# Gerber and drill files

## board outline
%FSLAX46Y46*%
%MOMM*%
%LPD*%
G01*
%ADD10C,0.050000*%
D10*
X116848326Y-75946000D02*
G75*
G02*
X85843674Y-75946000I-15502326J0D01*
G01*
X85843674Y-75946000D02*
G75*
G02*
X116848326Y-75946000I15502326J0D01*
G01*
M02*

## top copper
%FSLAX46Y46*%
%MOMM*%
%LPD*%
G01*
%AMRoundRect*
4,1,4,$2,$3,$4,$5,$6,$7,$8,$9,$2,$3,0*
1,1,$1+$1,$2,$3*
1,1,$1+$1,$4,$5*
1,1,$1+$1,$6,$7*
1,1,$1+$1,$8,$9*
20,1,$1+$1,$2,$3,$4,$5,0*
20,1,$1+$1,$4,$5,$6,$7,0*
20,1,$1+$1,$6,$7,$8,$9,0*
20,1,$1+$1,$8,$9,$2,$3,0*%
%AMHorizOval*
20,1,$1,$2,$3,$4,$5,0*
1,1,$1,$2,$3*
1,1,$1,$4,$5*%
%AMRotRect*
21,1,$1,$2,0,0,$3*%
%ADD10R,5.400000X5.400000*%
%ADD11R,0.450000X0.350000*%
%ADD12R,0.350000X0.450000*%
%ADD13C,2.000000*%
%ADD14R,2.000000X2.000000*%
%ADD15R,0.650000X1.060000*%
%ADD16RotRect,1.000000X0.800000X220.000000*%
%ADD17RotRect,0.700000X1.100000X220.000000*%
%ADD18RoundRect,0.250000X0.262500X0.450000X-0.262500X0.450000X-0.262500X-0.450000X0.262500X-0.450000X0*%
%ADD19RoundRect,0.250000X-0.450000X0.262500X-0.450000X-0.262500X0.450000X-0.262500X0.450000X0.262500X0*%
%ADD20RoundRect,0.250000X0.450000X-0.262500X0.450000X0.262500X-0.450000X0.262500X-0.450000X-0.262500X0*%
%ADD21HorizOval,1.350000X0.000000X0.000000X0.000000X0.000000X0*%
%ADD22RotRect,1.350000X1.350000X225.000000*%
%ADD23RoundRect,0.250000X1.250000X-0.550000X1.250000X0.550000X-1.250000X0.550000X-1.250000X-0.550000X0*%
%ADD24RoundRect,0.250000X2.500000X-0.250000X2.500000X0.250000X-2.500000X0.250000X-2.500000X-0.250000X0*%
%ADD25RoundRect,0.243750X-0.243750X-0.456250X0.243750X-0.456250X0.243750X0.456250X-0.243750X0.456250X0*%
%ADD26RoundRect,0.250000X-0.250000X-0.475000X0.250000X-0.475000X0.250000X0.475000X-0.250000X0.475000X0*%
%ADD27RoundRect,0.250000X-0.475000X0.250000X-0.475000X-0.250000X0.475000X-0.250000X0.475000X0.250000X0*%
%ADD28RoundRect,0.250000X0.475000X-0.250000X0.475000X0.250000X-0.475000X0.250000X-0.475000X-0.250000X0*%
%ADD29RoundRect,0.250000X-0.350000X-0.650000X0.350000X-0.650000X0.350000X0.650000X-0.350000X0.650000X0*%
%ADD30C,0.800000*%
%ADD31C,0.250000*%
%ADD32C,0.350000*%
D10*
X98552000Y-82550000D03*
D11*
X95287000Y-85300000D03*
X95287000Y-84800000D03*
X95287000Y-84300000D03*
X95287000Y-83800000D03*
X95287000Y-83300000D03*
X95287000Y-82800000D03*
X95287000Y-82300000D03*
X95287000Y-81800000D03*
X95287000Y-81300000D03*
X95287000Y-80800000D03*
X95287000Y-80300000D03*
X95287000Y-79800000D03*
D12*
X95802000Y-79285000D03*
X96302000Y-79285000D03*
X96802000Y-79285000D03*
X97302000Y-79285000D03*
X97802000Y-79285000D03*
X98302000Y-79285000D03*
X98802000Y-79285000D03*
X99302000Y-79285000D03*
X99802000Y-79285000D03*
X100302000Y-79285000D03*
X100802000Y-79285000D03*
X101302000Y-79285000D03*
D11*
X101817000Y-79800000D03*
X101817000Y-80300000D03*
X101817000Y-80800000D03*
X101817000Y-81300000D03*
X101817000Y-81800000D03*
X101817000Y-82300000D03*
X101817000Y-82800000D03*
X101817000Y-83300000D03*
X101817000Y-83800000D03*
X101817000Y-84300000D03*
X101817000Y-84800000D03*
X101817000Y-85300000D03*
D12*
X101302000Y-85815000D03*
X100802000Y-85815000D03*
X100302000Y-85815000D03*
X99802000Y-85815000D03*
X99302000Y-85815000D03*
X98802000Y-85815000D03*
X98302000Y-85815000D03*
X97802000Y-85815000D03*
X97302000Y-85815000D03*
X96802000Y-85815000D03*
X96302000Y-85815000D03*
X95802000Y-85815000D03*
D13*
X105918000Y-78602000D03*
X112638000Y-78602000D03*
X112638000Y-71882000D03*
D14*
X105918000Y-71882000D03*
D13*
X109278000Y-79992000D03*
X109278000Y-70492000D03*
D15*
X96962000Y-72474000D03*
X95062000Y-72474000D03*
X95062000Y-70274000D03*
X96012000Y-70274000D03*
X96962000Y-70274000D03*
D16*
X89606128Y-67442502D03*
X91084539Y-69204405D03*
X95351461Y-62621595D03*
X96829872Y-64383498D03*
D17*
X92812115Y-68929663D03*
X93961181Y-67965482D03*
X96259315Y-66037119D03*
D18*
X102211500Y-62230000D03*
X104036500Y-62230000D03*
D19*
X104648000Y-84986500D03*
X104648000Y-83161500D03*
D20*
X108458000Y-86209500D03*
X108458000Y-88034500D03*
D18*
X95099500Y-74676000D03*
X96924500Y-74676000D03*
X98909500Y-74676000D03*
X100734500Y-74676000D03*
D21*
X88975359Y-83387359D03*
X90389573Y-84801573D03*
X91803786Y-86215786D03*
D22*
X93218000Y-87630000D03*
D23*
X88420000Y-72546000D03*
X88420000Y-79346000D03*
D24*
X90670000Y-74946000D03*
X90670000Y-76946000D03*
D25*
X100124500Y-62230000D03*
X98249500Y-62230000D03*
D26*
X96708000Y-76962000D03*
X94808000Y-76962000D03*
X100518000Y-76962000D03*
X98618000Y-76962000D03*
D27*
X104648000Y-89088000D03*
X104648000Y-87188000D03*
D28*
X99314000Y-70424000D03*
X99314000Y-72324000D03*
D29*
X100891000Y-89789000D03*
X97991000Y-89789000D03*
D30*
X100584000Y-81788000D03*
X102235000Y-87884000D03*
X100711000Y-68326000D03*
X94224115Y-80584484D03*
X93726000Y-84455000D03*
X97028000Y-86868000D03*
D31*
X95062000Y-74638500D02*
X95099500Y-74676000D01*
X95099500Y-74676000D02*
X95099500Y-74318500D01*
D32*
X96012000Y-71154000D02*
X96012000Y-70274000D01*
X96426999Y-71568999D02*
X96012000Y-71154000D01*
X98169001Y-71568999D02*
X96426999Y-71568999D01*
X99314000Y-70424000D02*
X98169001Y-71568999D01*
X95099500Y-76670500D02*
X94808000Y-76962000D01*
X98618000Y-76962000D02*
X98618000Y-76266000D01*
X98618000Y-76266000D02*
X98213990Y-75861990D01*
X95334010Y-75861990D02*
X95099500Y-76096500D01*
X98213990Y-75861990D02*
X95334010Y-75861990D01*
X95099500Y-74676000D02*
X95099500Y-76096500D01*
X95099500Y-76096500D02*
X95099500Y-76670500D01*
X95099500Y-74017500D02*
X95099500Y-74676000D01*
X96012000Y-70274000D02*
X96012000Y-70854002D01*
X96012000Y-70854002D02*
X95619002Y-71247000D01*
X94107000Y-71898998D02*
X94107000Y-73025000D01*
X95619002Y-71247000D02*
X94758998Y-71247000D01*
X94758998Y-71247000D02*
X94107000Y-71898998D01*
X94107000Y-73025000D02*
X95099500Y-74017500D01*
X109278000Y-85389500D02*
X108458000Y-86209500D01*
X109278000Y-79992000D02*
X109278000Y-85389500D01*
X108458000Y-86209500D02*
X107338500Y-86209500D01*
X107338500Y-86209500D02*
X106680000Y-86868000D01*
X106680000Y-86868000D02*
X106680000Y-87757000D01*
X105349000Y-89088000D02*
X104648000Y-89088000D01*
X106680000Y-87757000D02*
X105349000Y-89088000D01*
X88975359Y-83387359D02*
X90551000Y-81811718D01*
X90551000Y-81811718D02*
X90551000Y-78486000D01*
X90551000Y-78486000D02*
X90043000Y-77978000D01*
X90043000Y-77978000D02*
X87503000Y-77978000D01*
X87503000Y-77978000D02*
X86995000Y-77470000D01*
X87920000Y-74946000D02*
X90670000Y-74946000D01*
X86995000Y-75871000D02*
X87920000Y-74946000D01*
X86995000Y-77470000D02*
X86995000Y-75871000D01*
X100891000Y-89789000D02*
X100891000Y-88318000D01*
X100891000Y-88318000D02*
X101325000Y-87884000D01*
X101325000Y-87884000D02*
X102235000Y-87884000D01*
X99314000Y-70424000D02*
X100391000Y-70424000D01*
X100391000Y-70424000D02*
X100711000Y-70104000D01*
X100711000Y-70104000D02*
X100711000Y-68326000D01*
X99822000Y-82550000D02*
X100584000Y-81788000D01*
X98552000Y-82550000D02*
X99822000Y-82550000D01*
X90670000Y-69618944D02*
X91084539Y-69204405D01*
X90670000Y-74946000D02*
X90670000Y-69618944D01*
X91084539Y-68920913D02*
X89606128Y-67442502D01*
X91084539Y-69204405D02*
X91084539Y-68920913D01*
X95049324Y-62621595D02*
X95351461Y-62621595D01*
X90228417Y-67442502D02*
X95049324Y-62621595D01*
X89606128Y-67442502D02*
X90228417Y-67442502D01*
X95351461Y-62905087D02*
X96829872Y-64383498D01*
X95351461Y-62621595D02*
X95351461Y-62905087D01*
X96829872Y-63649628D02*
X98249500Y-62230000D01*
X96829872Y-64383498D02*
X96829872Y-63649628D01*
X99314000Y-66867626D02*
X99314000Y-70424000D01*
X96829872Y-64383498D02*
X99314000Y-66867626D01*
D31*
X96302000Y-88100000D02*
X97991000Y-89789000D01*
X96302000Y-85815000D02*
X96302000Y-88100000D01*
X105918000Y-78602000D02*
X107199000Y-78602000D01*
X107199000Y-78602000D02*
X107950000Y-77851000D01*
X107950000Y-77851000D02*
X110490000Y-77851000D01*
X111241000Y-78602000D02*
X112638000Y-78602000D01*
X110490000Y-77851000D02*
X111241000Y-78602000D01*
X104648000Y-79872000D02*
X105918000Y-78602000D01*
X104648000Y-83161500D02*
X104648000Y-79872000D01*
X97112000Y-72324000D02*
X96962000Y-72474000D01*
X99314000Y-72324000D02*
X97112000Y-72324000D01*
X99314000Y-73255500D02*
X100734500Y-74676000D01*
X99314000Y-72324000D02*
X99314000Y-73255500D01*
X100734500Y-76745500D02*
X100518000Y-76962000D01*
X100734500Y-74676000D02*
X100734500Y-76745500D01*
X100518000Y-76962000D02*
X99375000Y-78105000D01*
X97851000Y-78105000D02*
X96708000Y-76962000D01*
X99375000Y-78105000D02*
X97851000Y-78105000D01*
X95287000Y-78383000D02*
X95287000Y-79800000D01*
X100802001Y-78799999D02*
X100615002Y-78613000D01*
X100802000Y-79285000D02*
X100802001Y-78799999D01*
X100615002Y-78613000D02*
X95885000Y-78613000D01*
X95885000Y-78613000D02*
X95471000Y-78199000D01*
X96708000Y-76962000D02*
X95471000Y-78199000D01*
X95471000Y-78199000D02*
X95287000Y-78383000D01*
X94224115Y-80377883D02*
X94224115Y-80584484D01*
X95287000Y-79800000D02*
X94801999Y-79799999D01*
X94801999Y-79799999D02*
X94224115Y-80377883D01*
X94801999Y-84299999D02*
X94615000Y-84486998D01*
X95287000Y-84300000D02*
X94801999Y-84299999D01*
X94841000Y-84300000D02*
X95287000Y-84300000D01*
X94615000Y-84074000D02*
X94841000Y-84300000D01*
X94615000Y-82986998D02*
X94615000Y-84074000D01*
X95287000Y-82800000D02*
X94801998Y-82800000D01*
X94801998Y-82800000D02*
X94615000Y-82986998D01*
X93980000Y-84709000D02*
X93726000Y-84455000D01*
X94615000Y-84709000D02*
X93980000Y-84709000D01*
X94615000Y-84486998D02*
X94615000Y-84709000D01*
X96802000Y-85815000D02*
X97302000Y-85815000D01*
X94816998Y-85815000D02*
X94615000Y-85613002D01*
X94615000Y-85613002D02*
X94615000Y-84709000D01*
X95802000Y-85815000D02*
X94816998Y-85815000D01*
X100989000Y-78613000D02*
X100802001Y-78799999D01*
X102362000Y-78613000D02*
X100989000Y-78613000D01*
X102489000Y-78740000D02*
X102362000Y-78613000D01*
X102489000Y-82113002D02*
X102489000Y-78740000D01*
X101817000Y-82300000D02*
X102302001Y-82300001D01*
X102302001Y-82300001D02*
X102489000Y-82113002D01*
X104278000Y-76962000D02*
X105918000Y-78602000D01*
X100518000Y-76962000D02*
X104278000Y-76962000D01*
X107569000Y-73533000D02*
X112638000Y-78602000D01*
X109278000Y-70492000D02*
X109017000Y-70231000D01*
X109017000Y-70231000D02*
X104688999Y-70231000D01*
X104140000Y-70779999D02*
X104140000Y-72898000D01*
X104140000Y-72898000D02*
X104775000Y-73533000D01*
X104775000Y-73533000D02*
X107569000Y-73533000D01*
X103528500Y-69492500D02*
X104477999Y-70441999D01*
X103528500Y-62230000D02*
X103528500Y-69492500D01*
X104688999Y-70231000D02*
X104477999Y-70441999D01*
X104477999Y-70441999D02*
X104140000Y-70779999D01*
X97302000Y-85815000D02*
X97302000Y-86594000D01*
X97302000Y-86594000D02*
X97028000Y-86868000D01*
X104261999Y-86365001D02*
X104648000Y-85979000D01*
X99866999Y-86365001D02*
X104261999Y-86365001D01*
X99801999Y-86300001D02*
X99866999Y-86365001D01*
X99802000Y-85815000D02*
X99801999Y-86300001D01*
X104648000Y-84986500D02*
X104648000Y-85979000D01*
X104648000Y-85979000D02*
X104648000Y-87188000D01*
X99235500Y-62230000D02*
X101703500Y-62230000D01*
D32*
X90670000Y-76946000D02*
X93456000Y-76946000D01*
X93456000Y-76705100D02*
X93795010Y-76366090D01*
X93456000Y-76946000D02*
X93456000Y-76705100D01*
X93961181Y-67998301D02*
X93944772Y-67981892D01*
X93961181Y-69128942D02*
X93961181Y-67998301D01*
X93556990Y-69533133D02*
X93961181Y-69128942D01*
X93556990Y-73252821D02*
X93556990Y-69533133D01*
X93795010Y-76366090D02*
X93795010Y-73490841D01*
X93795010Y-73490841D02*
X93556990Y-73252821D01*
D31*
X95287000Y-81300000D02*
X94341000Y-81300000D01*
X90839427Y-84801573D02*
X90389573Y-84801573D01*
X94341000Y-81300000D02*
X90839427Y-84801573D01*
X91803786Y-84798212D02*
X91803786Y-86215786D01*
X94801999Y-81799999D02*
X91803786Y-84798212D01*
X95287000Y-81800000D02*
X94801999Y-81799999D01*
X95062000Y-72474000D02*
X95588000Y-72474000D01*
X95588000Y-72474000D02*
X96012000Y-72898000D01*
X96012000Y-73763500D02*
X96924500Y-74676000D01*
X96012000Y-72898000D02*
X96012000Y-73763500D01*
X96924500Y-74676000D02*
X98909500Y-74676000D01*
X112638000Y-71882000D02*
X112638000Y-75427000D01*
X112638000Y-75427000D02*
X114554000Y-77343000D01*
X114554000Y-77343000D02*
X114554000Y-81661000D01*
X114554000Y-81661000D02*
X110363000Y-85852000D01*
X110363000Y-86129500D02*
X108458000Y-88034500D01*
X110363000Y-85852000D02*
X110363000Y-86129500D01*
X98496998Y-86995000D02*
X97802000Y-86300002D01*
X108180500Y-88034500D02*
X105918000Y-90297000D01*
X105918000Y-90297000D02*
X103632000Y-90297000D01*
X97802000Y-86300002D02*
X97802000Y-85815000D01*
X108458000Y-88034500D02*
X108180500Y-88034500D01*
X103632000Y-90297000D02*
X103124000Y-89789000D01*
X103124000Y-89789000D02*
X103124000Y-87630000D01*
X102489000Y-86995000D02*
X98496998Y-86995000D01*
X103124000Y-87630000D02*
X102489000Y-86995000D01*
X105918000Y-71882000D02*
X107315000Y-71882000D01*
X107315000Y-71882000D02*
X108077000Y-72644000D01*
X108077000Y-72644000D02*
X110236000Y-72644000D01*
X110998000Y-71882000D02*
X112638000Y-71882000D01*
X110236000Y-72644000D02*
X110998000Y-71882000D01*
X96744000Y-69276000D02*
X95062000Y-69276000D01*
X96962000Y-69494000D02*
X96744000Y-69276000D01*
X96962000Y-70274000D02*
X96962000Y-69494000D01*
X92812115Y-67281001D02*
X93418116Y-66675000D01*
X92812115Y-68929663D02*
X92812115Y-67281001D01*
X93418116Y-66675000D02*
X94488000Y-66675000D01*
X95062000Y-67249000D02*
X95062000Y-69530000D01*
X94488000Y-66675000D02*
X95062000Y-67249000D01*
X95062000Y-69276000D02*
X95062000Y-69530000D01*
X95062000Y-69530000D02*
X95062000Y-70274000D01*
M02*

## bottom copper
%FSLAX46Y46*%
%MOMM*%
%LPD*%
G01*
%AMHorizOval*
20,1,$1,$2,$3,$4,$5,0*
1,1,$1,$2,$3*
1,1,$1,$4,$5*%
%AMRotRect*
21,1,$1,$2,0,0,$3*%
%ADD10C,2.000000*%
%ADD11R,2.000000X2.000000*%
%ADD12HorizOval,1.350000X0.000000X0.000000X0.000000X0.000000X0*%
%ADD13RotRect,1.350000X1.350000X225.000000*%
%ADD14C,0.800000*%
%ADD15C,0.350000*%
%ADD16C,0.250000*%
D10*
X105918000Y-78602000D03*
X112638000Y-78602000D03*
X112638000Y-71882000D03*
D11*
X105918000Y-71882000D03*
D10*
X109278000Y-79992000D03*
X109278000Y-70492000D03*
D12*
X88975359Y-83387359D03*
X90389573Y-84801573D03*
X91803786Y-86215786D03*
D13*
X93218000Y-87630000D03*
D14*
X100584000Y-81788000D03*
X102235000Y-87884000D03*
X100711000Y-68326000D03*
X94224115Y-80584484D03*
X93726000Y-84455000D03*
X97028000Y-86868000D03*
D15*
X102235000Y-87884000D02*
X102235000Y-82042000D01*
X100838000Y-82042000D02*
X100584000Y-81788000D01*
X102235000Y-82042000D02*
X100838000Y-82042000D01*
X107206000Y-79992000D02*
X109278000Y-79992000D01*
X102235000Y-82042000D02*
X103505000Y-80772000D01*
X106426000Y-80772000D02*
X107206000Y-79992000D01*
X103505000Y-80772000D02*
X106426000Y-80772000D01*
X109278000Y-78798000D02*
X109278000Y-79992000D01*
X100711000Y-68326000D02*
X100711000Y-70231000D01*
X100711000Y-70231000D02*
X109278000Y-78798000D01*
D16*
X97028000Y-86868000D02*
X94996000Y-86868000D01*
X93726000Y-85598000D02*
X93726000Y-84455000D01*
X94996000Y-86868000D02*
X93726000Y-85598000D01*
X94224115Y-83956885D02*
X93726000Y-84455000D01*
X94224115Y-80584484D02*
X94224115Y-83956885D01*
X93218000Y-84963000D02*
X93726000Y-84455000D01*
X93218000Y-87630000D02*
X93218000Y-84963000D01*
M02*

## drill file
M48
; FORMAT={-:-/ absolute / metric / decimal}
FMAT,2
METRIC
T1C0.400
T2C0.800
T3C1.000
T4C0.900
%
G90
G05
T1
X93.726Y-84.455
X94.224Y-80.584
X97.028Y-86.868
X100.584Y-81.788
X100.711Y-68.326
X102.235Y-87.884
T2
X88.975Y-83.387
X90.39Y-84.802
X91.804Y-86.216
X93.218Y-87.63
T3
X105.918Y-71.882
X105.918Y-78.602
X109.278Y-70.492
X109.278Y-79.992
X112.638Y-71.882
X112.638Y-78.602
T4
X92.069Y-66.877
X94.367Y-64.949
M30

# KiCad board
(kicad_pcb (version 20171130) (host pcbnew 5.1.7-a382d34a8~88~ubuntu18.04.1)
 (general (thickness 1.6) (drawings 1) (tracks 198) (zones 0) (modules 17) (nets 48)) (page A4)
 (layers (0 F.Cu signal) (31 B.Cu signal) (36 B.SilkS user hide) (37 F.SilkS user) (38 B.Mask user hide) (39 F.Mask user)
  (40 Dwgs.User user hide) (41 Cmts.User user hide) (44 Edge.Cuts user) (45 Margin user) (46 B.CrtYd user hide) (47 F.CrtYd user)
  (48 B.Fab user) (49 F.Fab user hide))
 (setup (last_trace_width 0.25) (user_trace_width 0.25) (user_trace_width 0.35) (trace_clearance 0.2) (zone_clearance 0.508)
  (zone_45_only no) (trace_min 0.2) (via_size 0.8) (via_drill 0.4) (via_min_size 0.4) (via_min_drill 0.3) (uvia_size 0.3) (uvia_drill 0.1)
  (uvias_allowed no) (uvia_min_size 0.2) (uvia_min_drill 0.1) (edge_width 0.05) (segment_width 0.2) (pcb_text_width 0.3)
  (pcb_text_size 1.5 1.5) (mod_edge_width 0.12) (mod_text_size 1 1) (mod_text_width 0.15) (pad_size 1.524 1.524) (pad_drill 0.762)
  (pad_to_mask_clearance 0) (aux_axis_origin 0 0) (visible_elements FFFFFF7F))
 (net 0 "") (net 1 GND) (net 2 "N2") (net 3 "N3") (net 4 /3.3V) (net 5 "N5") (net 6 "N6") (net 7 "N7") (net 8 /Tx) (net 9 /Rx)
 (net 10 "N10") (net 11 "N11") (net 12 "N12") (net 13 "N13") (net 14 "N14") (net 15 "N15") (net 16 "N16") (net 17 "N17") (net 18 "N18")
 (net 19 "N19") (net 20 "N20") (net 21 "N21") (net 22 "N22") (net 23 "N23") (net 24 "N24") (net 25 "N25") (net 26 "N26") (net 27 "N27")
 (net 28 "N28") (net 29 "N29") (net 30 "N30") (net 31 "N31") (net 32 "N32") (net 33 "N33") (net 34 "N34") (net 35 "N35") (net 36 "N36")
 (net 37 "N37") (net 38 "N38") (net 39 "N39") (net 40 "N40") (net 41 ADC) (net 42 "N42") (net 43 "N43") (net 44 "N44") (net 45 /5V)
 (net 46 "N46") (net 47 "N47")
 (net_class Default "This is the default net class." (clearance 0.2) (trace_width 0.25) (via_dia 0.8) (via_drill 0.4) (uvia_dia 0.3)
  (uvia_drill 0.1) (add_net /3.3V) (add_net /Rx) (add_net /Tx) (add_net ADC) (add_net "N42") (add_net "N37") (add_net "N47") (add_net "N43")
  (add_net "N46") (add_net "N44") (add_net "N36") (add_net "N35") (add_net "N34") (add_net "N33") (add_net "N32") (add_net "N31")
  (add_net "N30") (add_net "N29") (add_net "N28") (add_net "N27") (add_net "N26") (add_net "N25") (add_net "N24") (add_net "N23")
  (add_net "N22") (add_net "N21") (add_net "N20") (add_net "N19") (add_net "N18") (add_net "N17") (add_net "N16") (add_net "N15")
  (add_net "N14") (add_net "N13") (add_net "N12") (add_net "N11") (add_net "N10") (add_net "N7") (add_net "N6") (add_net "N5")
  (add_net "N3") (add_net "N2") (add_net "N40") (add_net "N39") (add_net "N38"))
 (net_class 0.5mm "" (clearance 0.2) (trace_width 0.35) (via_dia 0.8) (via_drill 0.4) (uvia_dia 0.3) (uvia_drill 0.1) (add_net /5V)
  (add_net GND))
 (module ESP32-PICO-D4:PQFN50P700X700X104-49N (layer F.Cu) (at 98.552 82.55 90)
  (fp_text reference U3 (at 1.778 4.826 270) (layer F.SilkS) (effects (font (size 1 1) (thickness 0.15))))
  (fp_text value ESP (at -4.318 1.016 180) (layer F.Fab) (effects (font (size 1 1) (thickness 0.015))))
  (pad 49 smd rect (at 0 0 90) (size 5.4 5.4) (layers F.Cu F.Mask) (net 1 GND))
  (pad 48 smd rect (at -2.75 -3.265 90) (size 0.35 0.45) (layers F.Cu F.Paste F.Mask) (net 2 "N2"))
  (pad 47 smd rect (at -2.25 -3.265 90) (size 0.35 0.45) (layers F.Cu F.Paste F.Mask) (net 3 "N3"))
  (pad 46 smd rect (at -1.75 -3.265 90) (size 0.35 0.45) (layers F.Cu F.Paste F.Mask) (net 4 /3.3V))
  (pad 45 smd rect (at -1.25 -3.265 90) (size 0.35 0.45) (layers F.Cu F.Paste F.Mask) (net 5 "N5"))
  (pad 44 smd rect (at -0.75 -3.265 90) (size 0.35 0.45) (layers F.Cu F.Paste F.Mask) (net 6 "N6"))
  (pad 43 smd rect (at -0.25 -3.265 90) (size 0.35 0.45) (layers F.Cu F.Paste F.Mask) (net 4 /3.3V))
  (pad 42 smd rect (at 0.25 -3.265 90) (size 0.35 0.45) (layers F.Cu F.Paste F.Mask) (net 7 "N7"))
  (pad 41 smd rect (at 0.75 -3.265 90) (size 0.35 0.45) (layers F.Cu F.Paste F.Mask) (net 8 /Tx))
  (pad 40 smd rect (at 1.25 -3.265 90) (size 0.35 0.45) (layers F.Cu F.Paste F.Mask) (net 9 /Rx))
  (pad 39 smd rect (at 1.75 -3.265 90) (size 0.35 0.45) (layers F.Cu F.Paste F.Mask) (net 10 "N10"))
  (pad 38 smd rect (at 2.25 -3.265 90) (size 0.35 0.45) (layers F.Cu F.Paste F.Mask) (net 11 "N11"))
  (pad 37 smd rect (at 2.75 -3.265 90) (size 0.35 0.45) (layers F.Cu F.Paste F.Mask) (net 4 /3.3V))
  (pad 36 smd rect (at 3.265 -2.75 90) (size 0.45 0.35) (layers F.Cu F.Paste F.Mask) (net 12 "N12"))
  (pad 35 smd rect (at 3.265 -2.25 90) (size 0.45 0.35) (layers F.Cu F.Paste F.Mask) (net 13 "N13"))
  (pad 34 smd rect (at 3.265 -1.75 90) (size 0.45 0.35) (layers F.Cu F.Paste F.Mask) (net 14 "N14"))
  (pad 33 smd rect (at 3.265 -1.25 90) (size 0.45 0.35) (layers F.Cu F.Paste F.Mask) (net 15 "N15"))
  (pad 32 smd rect (at 3.265 -0.75 90) (size 0.45 0.35) (layers F.Cu F.Paste F.Mask) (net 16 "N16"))
  (pad 31 smd rect (at 3.265 -0.25 90) (size 0.45 0.35) (layers F.Cu F.Paste F.Mask) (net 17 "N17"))
  (pad 30 smd rect (at 3.265 0.25 90) (size 0.45 0.35) (layers F.Cu F.Paste F.Mask) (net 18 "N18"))
  (pad 29 smd rect (at 3.265 0.75 90) (size 0.45 0.35) (layers F.Cu F.Paste F.Mask) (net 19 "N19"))
  (pad 28 smd rect (at 3.265 1.25 90) (size 0.45 0.35) (layers F.Cu F.Paste F.Mask) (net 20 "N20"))
  (pad 27 smd rect (at 3.265 1.75 90) (size 0.45 0.35) (layers F.Cu F.Paste F.Mask) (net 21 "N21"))
  (pad 26 smd rect (at 3.265 2.25 90) (size 0.45 0.35) (layers F.Cu F.Paste F.Mask) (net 4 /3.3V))
  (pad 25 smd rect (at 3.265 2.75 90) (size 0.45 0.35) (layers F.Cu F.Paste F.Mask) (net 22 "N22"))
  (pad 24 smd rect (at 2.75 3.265 90) (size 0.35 0.45) (layers F.Cu F.Paste F.Mask) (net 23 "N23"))
  (pad 23 smd rect (at 2.25 3.265 90) (size 0.35 0.45) (layers F.Cu F.Paste F.Mask) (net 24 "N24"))
  (pad 22 smd rect (at 1.75 3.265 90) (size 0.35 0.45) (layers F.Cu F.Paste F.Mask) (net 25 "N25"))
  (pad 21 smd rect (at 1.25 3.265 90) (size 0.35 0.45) (layers F.Cu F.Paste F.Mask) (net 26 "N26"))
  (pad 20 smd rect (at 0.75 3.265 90) (size 0.35 0.45) (layers F.Cu F.Paste F.Mask) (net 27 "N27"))
  (pad 19 smd rect (at 0.25 3.265 90) (size 0.35 0.45) (layers F.Cu F.Paste F.Mask) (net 4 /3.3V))
  (pad 18 smd rect (at -0.25 3.265 90) (size 0.35 0.45) (layers F.Cu F.Paste F.Mask) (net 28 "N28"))
  (pad 17 smd rect (at -0.75 3.265 90) (size 0.35 0.45) (layers F.Cu F.Paste F.Mask) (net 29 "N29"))
  (pad 16 smd rect (at -1.25 3.265 90) (size 0.35 0.45) (layers F.Cu F.Paste F.Mask) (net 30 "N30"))
  (pad 15 smd rect (at -1.75 3.265 90) (size 0.35 0.45) (layers F.Cu F.Paste F.Mask) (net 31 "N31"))
  (pad 14 smd rect (at -2.25 3.265 90) (size 0.35 0.45) (layers F.Cu F.Paste F.Mask) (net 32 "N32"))
  (pad 13 smd rect (at -2.75 3.265 90) (size 0.35 0.45) (layers F.Cu F.Paste F.Mask) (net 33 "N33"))
  (pad 12 smd rect (at -3.265 2.75 90) (size 0.45 0.35) (layers F.Cu F.Paste F.Mask) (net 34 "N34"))
  (pad 11 smd rect (at -3.265 2.25 90) (size 0.45 0.35) (layers F.Cu F.Paste F.Mask) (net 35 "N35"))
  (pad 10 smd rect (at -3.265 1.75 90) (size 0.45 0.35) (layers F.Cu F.Paste F.Mask) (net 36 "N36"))
  (pad 9 smd rect (at -3.265 1.25 90) (size 0.45 0.35) (layers F.Cu F.Paste F.Mask) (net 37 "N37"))
  (pad 8 smd rect (at -3.265 0.75 90) (size 0.45 0.35) (layers F.Cu F.Paste F.Mask) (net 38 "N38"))
  (pad 7 smd rect (at -3.265 0.25 90) (size 0.45 0.35) (layers F.Cu F.Paste F.Mask) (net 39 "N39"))
  (pad 6 smd rect (at -3.265 -0.25 90) (size 0.45 0.35) (layers F.Cu F.Paste F.Mask) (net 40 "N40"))
  (pad 5 smd rect (at -3.265 -0.75 90) (size 0.45 0.35) (layers F.Cu F.Paste F.Mask) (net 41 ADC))
  (pad 4 smd rect (at -3.265 -1.25 90) (size 0.45 0.35) (layers F.Cu F.Paste F.Mask) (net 4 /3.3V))
  (pad 3 smd rect (at -3.265 -1.75 90) (size 0.45 0.35) (layers F.Cu F.Paste F.Mask) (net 4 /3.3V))
  (pad 2 smd rect (at -3.265 -2.25 90) (size 0.45 0.35) (layers F.Cu F.Paste F.Mask) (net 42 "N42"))
  (pad 1 smd rect (at -3.265 -2.75 90) (size 0.45 0.35) (layers F.Cu F.Paste F.Mask) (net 4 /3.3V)))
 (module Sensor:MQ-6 (layer B.Cu) (at 105.918 71.882 270)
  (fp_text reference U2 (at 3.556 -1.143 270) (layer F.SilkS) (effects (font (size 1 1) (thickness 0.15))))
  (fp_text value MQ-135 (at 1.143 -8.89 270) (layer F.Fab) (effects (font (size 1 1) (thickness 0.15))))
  (pad 6 thru_hole circle (at 6.72 0) (size 2 2) (drill 1) (layers *.Cu *.Mask) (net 4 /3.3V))
  (pad 4 thru_hole circle (at 6.72 -6.72 90) (size 2 2) (drill 1) (layers *.Cu *.Mask) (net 4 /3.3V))
  (pad 3 thru_hole circle (at 0 -6.72 180) (size 2 2) (drill 1) (layers *.Cu *.Mask) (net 41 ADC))
  (pad 1 thru_hole rect (at 0 0 270) (size 2 2) (drill 1) (layers *.Cu *.Mask) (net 41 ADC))
  (pad 5 thru_hole circle (at 8.11 -3.36 270) (size 2 2) (drill 1) (layers *.Cu *.Mask) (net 1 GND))
  (pad 2 thru_hole circle (at -1.39 -3.36 270) (size 2 2) (drill 1) (layers *.Cu *.Mask) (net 4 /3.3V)))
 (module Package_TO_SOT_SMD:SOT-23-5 (layer F.Cu) (at 96.012 71.374 270)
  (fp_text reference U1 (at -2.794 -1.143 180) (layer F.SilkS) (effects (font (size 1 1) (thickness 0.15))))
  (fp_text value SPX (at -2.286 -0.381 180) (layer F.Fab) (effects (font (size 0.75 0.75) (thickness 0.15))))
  (pad 5 smd rect (at 1.1 -0.95 270) (size 1.06 0.65) (layers F.Cu F.Paste F.Mask) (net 4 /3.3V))
  (pad 4 smd rect (at 1.1 0.95 270) (size 1.06 0.65) (layers F.Cu F.Paste F.Mask) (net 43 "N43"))
  (pad 3 smd rect (at -1.1 0.95 270) (size 1.06 0.65) (layers F.Cu F.Paste F.Mask) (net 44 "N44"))
  (pad 2 smd rect (at -1.1 0 270) (size 1.06 0.65) (layers F.Cu F.Paste F.Mask) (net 1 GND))
  (pad 1 smd rect (at -1.1 -0.95 270) (size 1.06 0.65) (layers F.Cu F.Paste F.Mask) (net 44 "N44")))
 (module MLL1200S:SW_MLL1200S (layer F.Cu) (at 93.218 65.913 220)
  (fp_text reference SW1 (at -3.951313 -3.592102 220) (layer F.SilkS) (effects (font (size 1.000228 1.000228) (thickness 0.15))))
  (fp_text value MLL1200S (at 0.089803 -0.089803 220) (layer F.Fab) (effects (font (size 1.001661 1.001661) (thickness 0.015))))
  (pad G4 smd rect (at 3.75 1.15 220) (size 1 0.8) (layers F.Cu F.Paste F.Mask) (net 1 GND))
  (pad G2 smd rect (at 3.75 -1.15 220) (size 1 0.8) (layers F.Cu F.Paste F.Mask) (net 1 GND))
  (pad G3 smd rect (at -3.75 1.15 220) (size 1 0.8) (layers F.Cu F.Paste F.Mask) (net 1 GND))
  (pad G1 smd rect (at -3.75 -1.15 220) (size 1 0.8) (layers F.Cu F.Paste F.Mask) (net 1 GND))
  (pad 3 smd rect (at 2.25 -2.05 220) (size 0.7 1.1) (layers F.Cu F.Paste F.Mask) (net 44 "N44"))
  (pad 2 smd rect (at 0.75 -2.05 220) (size 0.7 1.1) (layers F.Cu F.Paste F.Mask) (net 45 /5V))
  (pad 1 smd rect (at -2.25 -2.05 220) (size 0.7 1.1) (layers F.Cu F.Paste F.Mask) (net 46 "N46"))
  (pad None np_thru_hole circle (at 1.5 0 220) (size 0.9 0.9) (drill 0.9) (layers *.Cu *.Mask))
  (pad None np_thru_hole circle (at -1.5 0 220) (size 0.9 0.9) (drill 0.9) (layers *.Cu *.Mask)))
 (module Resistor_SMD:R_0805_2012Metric (layer F.Cu) (at 103.124 62.23 180)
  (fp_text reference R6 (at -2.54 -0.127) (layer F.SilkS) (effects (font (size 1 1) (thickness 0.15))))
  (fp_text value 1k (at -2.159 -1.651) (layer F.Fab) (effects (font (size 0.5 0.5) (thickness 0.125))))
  (pad 2 smd roundrect (at 0.9125 0 180) (size 1.025 1.4) (layers F.Cu F.Paste F.Mask) (roundrect_rratio 0.243902) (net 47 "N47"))
  (pad 1 smd roundrect (at -0.9125 0 180) (size 1.025 1.4) (layers F.Cu F.Paste F.Mask) (roundrect_rratio 0.243902) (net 4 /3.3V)))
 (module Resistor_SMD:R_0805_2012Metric (layer F.Cu) (at 104.648 84.074 270)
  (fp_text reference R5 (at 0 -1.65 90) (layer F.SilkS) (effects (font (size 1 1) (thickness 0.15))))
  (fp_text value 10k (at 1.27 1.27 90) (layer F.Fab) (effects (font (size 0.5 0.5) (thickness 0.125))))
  (pad 2 smd roundrect (at 0.9125 0 270) (size 1.025 1.4) (layers F.Cu F.Paste F.Mask) (roundrect_rratio 0.243902) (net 37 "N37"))
  (pad 1 smd roundrect (at -0.9125 0 270) (size 1.025 1.4) (layers F.Cu F.Paste F.Mask) (roundrect_rratio 0.243902) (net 4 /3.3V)))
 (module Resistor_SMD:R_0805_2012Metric (layer F.Cu) (at 108.458 87.122 90)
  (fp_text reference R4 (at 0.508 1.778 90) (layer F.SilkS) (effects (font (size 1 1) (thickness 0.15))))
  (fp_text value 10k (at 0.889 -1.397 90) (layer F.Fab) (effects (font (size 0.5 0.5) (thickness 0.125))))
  (pad 2 smd roundrect (at 0.9125 0 90) (size 1.025 1.4) (layers F.Cu F.Paste F.Mask) (roundrect_rratio 0.243902) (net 1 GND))
  (pad 1 smd roundrect (at -0.9125 0 90) (size 1.025 1.4) (layers F.Cu F.Paste F.Mask) (roundrect_rratio 0.243902) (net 41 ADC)))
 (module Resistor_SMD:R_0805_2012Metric (layer F.Cu) (at 96.012 74.676 180)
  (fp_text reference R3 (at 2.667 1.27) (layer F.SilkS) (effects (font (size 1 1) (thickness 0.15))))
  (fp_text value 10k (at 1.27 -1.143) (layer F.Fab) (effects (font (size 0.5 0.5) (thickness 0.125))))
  (pad 2 smd roundrect (at 0.9125 0 180) (size 1.025 1.4) (layers F.Cu F.Paste F.Mask) (roundrect_rratio 0.243902) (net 1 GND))
  (pad 1 smd roundrect (at -0.9125 0 180) (size 1.025 1.4) (layers F.Cu F.Paste F.Mask) (roundrect_rratio 0.243902) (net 43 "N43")))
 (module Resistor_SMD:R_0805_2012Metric (layer F.Cu) (at 99.822 74.676 180)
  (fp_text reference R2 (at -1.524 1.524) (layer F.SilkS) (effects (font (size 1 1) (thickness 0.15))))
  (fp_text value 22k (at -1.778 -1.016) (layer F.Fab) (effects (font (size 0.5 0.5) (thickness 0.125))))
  (pad 2 smd roundrect (at 0.9125 0 180) (size 1.025 1.4) (layers F.Cu F.Paste F.Mask) (roundrect_rratio 0.243902) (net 43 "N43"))
  (pad 1 smd roundrect (at -0.9125 0 180) (size 1.025 1.4) (layers F.Cu F.Paste F.Mask) (roundrect_rratio 0.243902) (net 4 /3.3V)))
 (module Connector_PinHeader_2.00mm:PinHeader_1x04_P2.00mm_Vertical (layer F.Cu) (at 93.218 87.63 225)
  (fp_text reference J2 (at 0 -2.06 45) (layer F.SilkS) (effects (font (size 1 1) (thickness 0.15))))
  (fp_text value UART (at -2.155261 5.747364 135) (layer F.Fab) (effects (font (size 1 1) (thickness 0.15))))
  (pad 4 thru_hole oval (at 0 6 225) (size 1.35 1.35) (drill 0.8) (layers *.Cu *.Mask) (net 1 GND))
  (pad 3 thru_hole oval (at 0 4 225) (size 1.35 1.35) (drill 0.8) (layers *.Cu *.Mask) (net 9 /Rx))
  (pad 2 thru_hole oval (at 0 2 225) (size 1.35 1.35) (drill 0.8) (layers *.Cu *.Mask) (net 8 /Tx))
  (pad 1 thru_hole rect (at 0 0 225) (size 1.35 1.35) (drill 0.8) (layers *.Cu *.Mask) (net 4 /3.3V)))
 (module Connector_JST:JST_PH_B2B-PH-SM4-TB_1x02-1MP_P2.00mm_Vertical (layer F.Cu) (at 90.17 75.946 90)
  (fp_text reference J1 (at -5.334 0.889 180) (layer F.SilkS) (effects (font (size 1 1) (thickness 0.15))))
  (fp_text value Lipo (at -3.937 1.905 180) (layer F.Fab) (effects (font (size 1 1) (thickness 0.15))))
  (pad MP smd roundrect (at 3.4 -1.75 90) (size 1.6 3) (layers F.Cu F.Paste F.Mask) (roundrect_rratio 0.15625))
  (pad MP smd roundrect (at -3.4 -1.75 90) (size 1.6 3) (layers F.Cu F.Paste F.Mask) (roundrect_rratio 0.15625))
  (pad 2 smd roundrect (at 1 0.5 90) (size 1 5.5) (layers F.Cu F.Paste F.Mask) (roundrect_rratio 0.25) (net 1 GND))
  (pad 1 smd roundrect (at -1 0.5 90) (size 1 5.5) (layers F.Cu F.Paste F.Mask) (roundrect_rratio 0.25) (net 45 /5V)))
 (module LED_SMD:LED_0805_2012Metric (layer F.Cu) (at 99.187 62.23)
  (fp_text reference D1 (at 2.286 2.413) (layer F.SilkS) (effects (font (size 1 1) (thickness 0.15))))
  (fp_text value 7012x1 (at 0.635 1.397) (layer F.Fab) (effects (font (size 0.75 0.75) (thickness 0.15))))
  (pad 2 smd roundrect (at 0.9375 0) (size 0.975 1.4) (layers F.Cu F.Paste F.Mask) (roundrect_rratio 0.25) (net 47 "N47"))
  (pad 1 smd roundrect (at -0.9375 0) (size 0.975 1.4) (layers F.Cu F.Paste F.Mask) (roundrect_rratio 0.25) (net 1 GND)))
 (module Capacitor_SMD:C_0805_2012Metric (layer F.Cu) (at 95.758 76.962)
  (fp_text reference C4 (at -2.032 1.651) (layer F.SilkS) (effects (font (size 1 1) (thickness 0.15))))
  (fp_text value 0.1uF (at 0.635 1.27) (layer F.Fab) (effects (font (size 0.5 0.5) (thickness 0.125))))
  (pad 2 smd roundrect (at 0.95 0) (size 1 1.45) (layers F.Cu F.Paste F.Mask) (roundrect_rratio 0.25) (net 4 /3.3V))
  (pad 1 smd roundrect (at -0.95 0) (size 1 1.45) (layers F.Cu F.Paste F.Mask) (roundrect_rratio 0.25) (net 1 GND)))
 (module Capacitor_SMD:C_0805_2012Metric (layer F.Cu) (at 99.568 76.962)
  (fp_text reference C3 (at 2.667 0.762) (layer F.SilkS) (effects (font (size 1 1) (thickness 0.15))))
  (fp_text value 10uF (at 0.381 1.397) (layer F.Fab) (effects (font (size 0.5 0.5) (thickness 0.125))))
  (pad 2 smd roundrect (at 0.95 0) (size 1 1.45) (layers F.Cu F.Paste F.Mask) (roundrect_rratio 0.25) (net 4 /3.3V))
  (pad 1 smd roundrect (at -0.95 0) (size 1 1.45) (layers F.Cu F.Paste F.Mask) (roundrect_rratio 0.25) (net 1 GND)))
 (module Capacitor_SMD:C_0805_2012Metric (layer F.Cu) (at 104.648 88.138 270)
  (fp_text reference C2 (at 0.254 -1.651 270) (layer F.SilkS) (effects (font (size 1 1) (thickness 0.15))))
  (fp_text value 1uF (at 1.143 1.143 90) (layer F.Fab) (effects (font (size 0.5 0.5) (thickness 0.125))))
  (pad 2 smd roundrect (at 0.95 0 270) (size 1 1.45) (layers F.Cu F.Paste F.Mask) (roundrect_rratio 0.25) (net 1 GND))
  (pad 1 smd roundrect (at -0.95 0 270) (size 1 1.45) (layers F.Cu F.Paste F.Mask) (roundrect_rratio 0.25) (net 37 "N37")))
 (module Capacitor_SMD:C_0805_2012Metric (layer F.Cu) (at 99.314 71.374 90)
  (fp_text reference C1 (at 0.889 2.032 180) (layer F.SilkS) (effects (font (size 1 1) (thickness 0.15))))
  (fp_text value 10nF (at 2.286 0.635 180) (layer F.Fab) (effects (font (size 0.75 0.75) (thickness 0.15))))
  (pad 2 smd roundrect (at 0.95 0 90) (size 1 1.45) (layers F.Cu F.Paste F.Mask) (roundrect_rratio 0.25) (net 1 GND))
  (pad 1 smd roundrect (at -0.95 0 90) (size 1 1.45) (layers F.Cu F.Paste F.Mask) (roundrect_rratio 0.25) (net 4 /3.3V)))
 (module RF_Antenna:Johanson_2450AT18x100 (layer F.Cu) (at 99.441 89.789)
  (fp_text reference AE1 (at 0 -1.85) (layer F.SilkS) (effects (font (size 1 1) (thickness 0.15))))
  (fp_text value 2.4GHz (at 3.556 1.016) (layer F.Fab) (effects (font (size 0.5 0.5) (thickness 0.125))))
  (pad 2 smd roundrect (at 1.45 0) (size 1.2 1.8) (layers F.Cu F.Paste F.Mask) (roundrect_rratio 0.208333) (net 1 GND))
  (pad 1 smd roundrect (at -1.45 0) (size 1.2 1.8) (layers F.Cu F.Paste F.Mask) (roundrect_rratio 0.208333) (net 42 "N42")))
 (gr_circle (center 101.346 75.946) (end 85.852 76.454) (layer Edge.Cuts) (width 0.05))
 (via (at 100.584 81.788) (size 0.8) (drill 0.4) (layers F.Cu B.Cu) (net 1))
 (segment (start 95.062 74.6385) (end 95.0995 74.676) (width 0.25) (layer F.Cu) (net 1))
 (segment (start 95.0995 74.676) (end 95.0995 74.3185) (width 0.25) (layer F.Cu) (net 1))
 (segment (start 96.012 71.154) (end 96.012 70.274) (width 0.35) (layer F.Cu) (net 1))
 (segment (start 96.426999 71.568999) (end 96.012 71.154) (width 0.35) (layer F.Cu) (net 1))
 (segment (start 98.169001 71.568999) (end 96.426999 71.568999) (width 0.35) (layer F.Cu) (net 1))
 (segment (start 99.314 70.424) (end 98.169001 71.568999) (width 0.35) (layer F.Cu) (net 1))
 (segment (start 95.0995 76.6705) (end 94.808 76.962) (width 0.35) (layer F.Cu) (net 1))
 (segment (start 98.618 76.962) (end 98.618 76.266) (width 0.35) (layer F.Cu) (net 1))
 (segment (start 98.618 76.266) (end 98.21399 75.86199) (width 0.35) (layer F.Cu) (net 1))
 (segment (start 95.33401 75.86199) (end 95.0995 76.0965) (width 0.35) (layer F.Cu) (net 1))
 (segment (start 98.21399 75.86199) (end 95.33401 75.86199) (width 0.35) (layer F.Cu) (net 1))
 (segment (start 95.0995 74.676) (end 95.0995 76.0965) (width 0.35) (layer F.Cu) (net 1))
 (segment (start 95.0995 76.0965) (end 95.0995 76.6705) (width 0.35) (layer F.Cu) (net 1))
 (segment (start 95.0995 74.0175) (end 95.0995 74.676) (width 0.35) (layer F.Cu) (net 1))
 (segment (start 96.012 70.274) (end 96.012 70.854002) (width 0.35) (layer F.Cu) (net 1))
 (segment (start 96.012 70.854002) (end 95.619002 71.247) (width 0.35) (layer F.Cu) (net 1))
 (segment (start 94.107 71.898998) (end 94.107 73.025) (width 0.35) (layer F.Cu) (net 1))
 (segment (start 95.619002 71.247) (end 94.758998 71.247) (width 0.35) (layer F.Cu) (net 1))
 (segment (start 94.758998 71.247) (end 94.107 71.898998) (width 0.35) (layer F.Cu) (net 1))
 (segment (start 94.107 73.025) (end 95.0995 74.0175) (width 0.35) (layer F.Cu) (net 1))
 (segment (start 109.278 85.3895) (end 108.458 86.2095) (width 0.35) (layer F.Cu) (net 1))
 (segment (start 109.278 79.992) (end 109.278 85.3895) (width 0.35) (layer F.Cu) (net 1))
 (segment (start 108.458 86.2095) (end 107.3385 86.2095) (width 0.35) (layer F.Cu) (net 1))
 (segment (start 107.3385 86.2095) (end 106.68 86.868) (width 0.35) (layer F.Cu) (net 1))
 (segment (start 106.68 86.868) (end 106.68 87.757) (width 0.35) (layer F.Cu) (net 1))
 (segment (start 105.349 89.088) (end 104.648 89.088) (width 0.35) (layer F.Cu) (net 1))
 (segment (start 106.68 87.757) (end 105.349 89.088) (width 0.35) (layer F.Cu) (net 1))
 (segment (start 88.975359 83.387359) (end 90.551 81.811718) (width 0.35) (layer F.Cu) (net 1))
 (segment (start 90.551 81.811718) (end 90.551 78.486) (width 0.35) (layer F.Cu) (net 1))
 (segment (start 90.551 78.486) (end 90.043 77.978) (width 0.35) (layer F.Cu) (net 1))
 (segment (start 90.043 77.978) (end 87.503 77.978) (width 0.35) (layer F.Cu) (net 1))
 (segment (start 87.503 77.978) (end 86.995 77.47) (width 0.35) (layer F.Cu) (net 1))
 (segment (start 87.92 74.946) (end 90.67 74.946) (width 0.35) (layer F.Cu) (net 1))
 (segment (start 86.995 75.871) (end 87.92 74.946) (width 0.35) (layer F.Cu) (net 1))
 (segment (start 86.995 77.47) (end 86.995 75.871) (width 0.35) (layer F.Cu) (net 1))
 (segment (start 100.891 89.789) (end 100.891 88.318) (width 0.35) (layer F.Cu) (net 1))
 (via (at 102.235 87.884) (size 0.8) (drill 0.4) (layers F.Cu B.Cu) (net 1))
 (segment (start 100.891 88.318) (end 101.325 87.884) (width 0.35) (layer F.Cu) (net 1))
 (segment (start 101.325 87.884) (end 102.235 87.884) (width 0.35) (layer F.Cu) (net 1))
 (segment (start 102.235 87.884) (end 102.235 82.042) (width 0.35) (layer B.Cu) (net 1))
 (segment (start 99.314 70.424) (end 100.391 70.424) (width 0.35) (layer F.Cu) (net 1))
 (via (at 100.711 68.326) (size 0.8) (drill 0.4) (layers F.Cu B.Cu) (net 1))
 (segment (start 100.391 70.424) (end 100.711 70.104) (width 0.35) (layer F.Cu) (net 1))
 (segment (start 100.711 70.104) (end 100.711 68.326) (width 0.35) (layer F.Cu) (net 1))
 (segment (start 99.822 82.55) (end 100.584 81.788) (width 0.35) (layer F.Cu) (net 1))
 (segment (start 98.552 82.55) (end 99.822 82.55) (width 0.35) (layer F.Cu) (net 1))
 (segment (start 100.838 82.042) (end 100.584 81.788) (width 0.35) (layer B.Cu) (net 1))
 (segment (start 102.235 82.042) (end 100.838 82.042) (width 0.35) (layer B.Cu) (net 1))
 (segment (start 107.206 79.992) (end 109.278 79.992) (width 0.35) (layer B.Cu) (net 1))
 (segment (start 102.235 82.042) (end 103.505 80.772) (width 0.35) (layer B.Cu) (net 1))
 (segment (start 106.426 80.772) (end 107.206 79.992) (width 0.35) (layer B.Cu) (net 1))
 (segment (start 103.505 80.772) (end 106.426 80.772) (width 0.35) (layer B.Cu) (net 1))
 (segment (start 109.278 78.798) (end 109.278 79.992) (width 0.35) (layer B.Cu) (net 1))
 (segment (start 100.711 68.326) (end 100.711 70.231) (width 0.35) (layer B.Cu) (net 1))
 (segment (start 100.711 70.231) (end 109.278 78.798) (width 0.35) (layer B.Cu) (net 1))
 (segment (start 90.67 69.618944) (end 91.084539 69.204405) (width 0.35) (layer F.Cu) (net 1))
 (segment (start 90.67 74.946) (end 90.67 69.618944) (width 0.35) (layer F.Cu) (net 1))
 (segment (start 91.084539 68.920913) (end 89.606128 67.442502) (width 0.35) (layer F.Cu) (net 1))
 (segment (start 91.084539 69.204405) (end 91.084539 68.920913) (width 0.35) (layer F.Cu) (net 1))
 (segment (start 95.049324 62.621595) (end 95.351461 62.621595) (width 0.35) (layer F.Cu) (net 1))
 (segment (start 90.228417 67.442502) (end 95.049324 62.621595) (width 0.35) (layer F.Cu) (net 1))
 (segment (start 89.606128 67.442502) (end 90.228417 67.442502) (width 0.35) (layer F.Cu) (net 1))
 (segment (start 95.351461 62.905087) (end 96.829872 64.383498) (width 0.35) (layer F.Cu) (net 1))
 (segment (start 95.351461 62.621595) (end 95.351461 62.905087) (width 0.35) (layer F.Cu) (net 1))
 (segment (start 96.829872 63.649628) (end 98.2495 62.23) (width 0.35) (layer F.Cu) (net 1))
 (segment (start 96.829872 64.383498) (end 96.829872 63.649628) (width 0.35) (layer F.Cu) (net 1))
 (segment (start 99.314 66.867626) (end 99.314 70.424) (width 0.35) (layer F.Cu) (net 1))
 (segment (start 96.829872 64.383498) (end 99.314 66.867626) (width 0.35) (layer F.Cu) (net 1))
 (segment (start 96.302 88.1) (end 97.991 89.789) (width 0.25) (layer F.Cu) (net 42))
 (segment (start 96.302 85.815) (end 96.302 88.1) (width 0.25) (layer F.Cu) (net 42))
 (segment (start 105.918 78.602) (end 107.199 78.602) (width 0.25) (layer F.Cu) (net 4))
 (segment (start 107.199 78.602) (end 107.95 77.851) (width 0.25) (layer F.Cu) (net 4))
 (segment (start 107.95 77.851) (end 110.49 77.851) (width 0.25) (layer F.Cu) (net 4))
 (segment (start 111.241 78.602) (end 112.638 78.602) (width 0.25) (layer F.Cu) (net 4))
 (segment (start 110.49 77.851) (end 111.241 78.602) (width 0.25) (layer F.Cu) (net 4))
 (segment (start 104.648 79.872) (end 105.918 78.602) (width 0.25) (layer F.Cu) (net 4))
 (segment (start 104.648 83.1615) (end 104.648 79.872) (width 0.25) (layer F.Cu) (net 4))
 (segment (start 97.112 72.324) (end 96.962 72.474) (width 0.25) (layer F.Cu) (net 4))
 (segment (start 99.314 72.324) (end 97.112 72.324) (width 0.25) (layer F.Cu) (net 4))
 (segment (start 99.314 73.2555) (end 100.7345 74.676) (width 0.25) (layer F.Cu) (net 4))
 (segment (start 99.314 72.324) (end 99.314 73.2555) (width 0.25) (layer F.Cu) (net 4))
 (segment (start 100.7345 76.7455) (end 100.518 76.962) (width 0.25) (layer F.Cu) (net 4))
 (segment (start 100.7345 74.676) (end 100.7345 76.7455) (width 0.25) (layer F.Cu) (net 4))
 (segment (start 100.518 76.962) (end 99.375 78.105) (width 0.25) (layer F.Cu) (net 4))
 (segment (start 97.851 78.105) (end 96.708 76.962) (width 0.25) (layer F.Cu) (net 4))
 (segment (start 99.375 78.105) (end 97.851 78.105) (width 0.25) (layer F.Cu) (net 4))
 (segment (start 95.287 78.383) (end 95.287 79.8) (width 0.25) (layer F.Cu) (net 4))
 (segment (start 100.802001 78.799999) (end 100.615002 78.613) (width 0.25) (layer F.Cu) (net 4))
 (segment (start 100.802 79.285) (end 100.802001 78.799999) (width 0.25) (layer F.Cu) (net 4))
 (segment (start 100.615002 78.613) (end 95.885 78.613) (width 0.25) (layer F.Cu) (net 4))
 (segment (start 95.885 78.613) (end 95.471 78.199) (width 0.25) (layer F.Cu) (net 4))
 (segment (start 96.708 76.962) (end 95.471 78.199) (width 0.25) (layer F.Cu) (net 4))
 (segment (start 95.471 78.199) (end 95.287 78.383) (width 0.25) (layer F.Cu) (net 4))
 (via (at 94.224115 80.584484) (size 0.8) (drill 0.4) (layers F.Cu B.Cu) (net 4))
 (segment (start 94.224115 80.377883) (end 94.224115 80.584484) (width 0.25) (layer F.Cu) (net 4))
 (segment (start 95.287 79.8) (end 94.801999 79.799999) (width 0.25) (layer F.Cu) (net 4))
 (segment (start 94.801999 79.799999) (end 94.224115 80.377883) (width 0.25) (layer F.Cu) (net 4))
 (segment (start 94.801999 84.299999) (end 94.615 84.486998) (width 0.25) (layer F.Cu) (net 4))
 (segment (start 95.287 84.3) (end 94.801999 84.299999) (width 0.25) (layer F.Cu) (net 4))
 (segment (start 94.841 84.3) (end 95.287 84.3) (width 0.25) (layer F.Cu) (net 4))
 (segment (start 94.615 84.074) (end 94.841 84.3) (width 0.25) (layer F.Cu) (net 4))
 (segment (start 94.615 82.986998) (end 94.615 84.074) (width 0.25) (layer F.Cu) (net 4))
 (segment (start 95.287 82.8) (end 94.801998 82.8) (width 0.25) (layer F.Cu) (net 4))
 (segment (start 94.801998 82.8) (end 94.615 82.986998) (width 0.25) (layer F.Cu) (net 4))
 (via (at 93.726 84.455) (size 0.8) (drill 0.4) (layers F.Cu B.Cu) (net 4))
 (segment (start 93.98 84.709) (end 93.726 84.455) (width 0.25) (layer F.Cu) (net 4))
 (segment (start 94.615 84.709) (end 93.98 84.709) (width 0.25) (layer F.Cu) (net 4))
 (segment (start 94.615 84.486998) (end 94.615 84.709) (width 0.25) (layer F.Cu) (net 4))
 (segment (start 96.802 85.815) (end 97.302 85.815) (width 0.25) (layer F.Cu) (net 4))
 (segment (start 94.816998 85.815) (end 94.615 85.613002) (width 0.25) (layer F.Cu) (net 4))
 (segment (start 94.615 85.613002) (end 94.615 84.709) (width 0.25) (layer F.Cu) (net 4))
 (segment (start 95.802 85.815) (end 94.816998 85.815) (width 0.25) (layer F.Cu) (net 4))
 (segment (start 100.989 78.613) (end 100.802001 78.799999) (width 0.25) (layer F.Cu) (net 4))
 (segment (start 102.362 78.613) (end 100.989 78.613) (width 0.25) (layer F.Cu) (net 4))
 (segment (start 102.489 78.74) (end 102.362 78.613) (width 0.25) (layer F.Cu) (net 4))
 (segment (start 102.489 82.113002) (end 102.489 78.74) (width 0.25) (layer F.Cu) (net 4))
 (segment (start 101.817 82.3) (end 102.302001 82.300001) (width 0.25) (layer F.Cu) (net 4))
 (segment (start 102.302001 82.300001) (end 102.489 82.113002) (width 0.25) (layer F.Cu) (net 4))
 (segment (start 104.278 76.962) (end 105.918 78.602) (width 0.25) (layer F.Cu) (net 4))
 (segment (start 100.518 76.962) (end 104.278 76.962) (width 0.25) (layer F.Cu) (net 4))
 (segment (start 107.569 73.533) (end 112.638 78.602) (width 0.25) (layer F.Cu) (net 4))
 (segment (start 109.278 70.492) (end 109.017 70.231) (width 0.25) (layer F.Cu) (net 4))
 (segment (start 109.017 70.231) (end 104.688999 70.231) (width 0.25) (layer F.Cu) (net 4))
 (segment (start 104.14 70.779999) (end 104.14 72.898) (width 0.25) (layer F.Cu) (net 4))
 (segment (start 104.14 72.898) (end 104.775 73.533) (width 0.25) (layer F.Cu) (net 4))
 (segment (start 104.775 73.533) (end 107.569 73.533) (width 0.25) (layer F.Cu) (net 4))
 (segment (start 103.5285 69.4925) (end 104.477999 70.441999) (width 0.25) (layer F.Cu) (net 4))
 (segment (start 103.5285 62.23) (end 103.5285 69.4925) (width 0.25) (layer F.Cu) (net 4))
 (segment (start 104.688999 70.231) (end 104.477999 70.441999) (width 0.25) (layer F.Cu) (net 4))
 (segment (start 104.477999 70.441999) (end 104.14 70.779999) (width 0.25) (layer F.Cu) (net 4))
 (via (at 97.028 86.868) (size 0.8) (drill 0.4) (layers F.Cu B.Cu) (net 4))
 (segment (start 97.302 85.815) (end 97.302 86.594) (width 0.25) (layer F.Cu) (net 4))
 (segment (start 97.302 86.594) (end 97.028 86.868) (width 0.25) (layer F.Cu) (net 4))
 (segment (start 97.028 86.868) (end 94.996 86.868) (width 0.25) (layer B.Cu) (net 4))
 (segment (start 93.726 85.598) (end 93.726 84.455) (width 0.25) (layer B.Cu) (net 4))
 (segment (start 94.996 86.868) (end 93.726 85.598) (width 0.25) (layer B.Cu) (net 4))
 (segment (start 94.224115 83.956885) (end 93.726 84.455) (width 0.25) (layer B.Cu) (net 4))
 (segment (start 94.224115 80.584484) (end 94.224115 83.956885) (width 0.25) (layer B.Cu) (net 4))
 (segment (start 93.218 84.963) (end 93.726 84.455) (width 0.25) (layer B.Cu) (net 4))
 (segment (start 93.218 87.63) (end 93.218 84.963) (width 0.25) (layer B.Cu) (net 4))
 (segment (start 104.261999 86.365001) (end 104.648 85.979) (width 0.25) (layer F.Cu) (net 37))
 (segment (start 99.866999 86.365001) (end 104.261999 86.365001) (width 0.25) (layer F.Cu) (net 37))
 (segment (start 99.801999 86.300001) (end 99.866999 86.365001) (width 0.25) (layer F.Cu) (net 37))
 (segment (start 99.802 85.815) (end 99.801999 86.300001) (width 0.25) (layer F.Cu) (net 37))
 (segment (start 104.648 84.9865) (end 104.648 85.979) (width 0.25) (layer F.Cu) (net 37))
 (segment (start 104.648 85.979) (end 104.648 87.188) (width 0.25) (layer F.Cu) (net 37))
 (segment (start 99.2355 62.23) (end 101.7035 62.23) (width 0.25) (layer F.Cu) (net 47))
 (segment (start 90.67 76.946) (end 93.456 76.946) (width 0.35) (layer F.Cu) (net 45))
 (segment (start 93.456 76.7051) (end 93.79501 76.36609) (width 0.35) (layer F.Cu) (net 45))
 (segment (start 93.456 76.946) (end 93.456 76.7051) (width 0.35) (layer F.Cu) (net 45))
 (segment (start 93.961181 67.998301) (end 93.944772 67.981892) (width 0.35) (layer F.Cu) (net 45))
 (segment (start 93.961181 69.128942) (end 93.961181 67.998301) (width 0.35) (layer F.Cu) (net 45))
 (segment (start 93.55699 69.533133) (end 93.961181 69.128942) (width 0.35) (layer F.Cu) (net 45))
 (segment (start 93.55699 73.252821) (end 93.55699 69.533133) (width 0.35) (layer F.Cu) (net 45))
 (segment (start 93.79501 76.36609) (end 93.79501 73.490841) (width 0.35) (layer F.Cu) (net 45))
 (segment (start 93.79501 73.490841) (end 93.55699 73.252821) (width 0.35) (layer F.Cu) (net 45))
 (segment (start 95.287 81.3) (end 94.341 81.3) (width 0.25) (layer F.Cu) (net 9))
 (segment (start 90.839427 84.801573) (end 90.389573 84.801573) (width 0.25) (layer F.Cu) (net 9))
 (segment (start 94.341 81.3) (end 90.839427 84.801573) (width 0.25) (layer F.Cu) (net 9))
 (segment (start 91.803786 84.798212) (end 91.803786 86.215786) (width 0.25) (layer F.Cu) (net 8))
 (segment (start 94.801999 81.799999) (end 91.803786 84.798212) (width 0.25) (layer F.Cu) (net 8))
 (segment (start 95.287 81.8) (end 94.801999 81.799999) (width 0.25) (layer F.Cu) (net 8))
 (segment (start 95.062 72.474) (end 95.588 72.474) (width 0.25) (layer F.Cu) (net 43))
 (segment (start 95.588 72.474) (end 96.012 72.898) (width 0.25) (layer F.Cu) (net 43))
 (segment (start 96.012 73.7635) (end 96.9245 74.676) (width 0.25) (layer F.Cu) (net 43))
 (segment (start 96.012 72.898) (end 96.012 73.7635) (width 0.25) (layer F.Cu) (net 43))
 (segment (start 96.9245 74.676) (end 98.9095 74.676) (width 0.25) (layer F.Cu) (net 43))
 (segment (start 112.638 71.882) (end 112.638 75.427) (width 0.25) (layer F.Cu) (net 41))
 (segment (start 112.638 75.427) (end 114.554 77.343) (width 0.25) (layer F.Cu) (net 41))
 (segment (start 114.554 77.343) (end 114.554 81.661) (width 0.25) (layer F.Cu) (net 41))
 (segment (start 114.554 81.661) (end 110.363 85.852) (width 0.25) (layer F.Cu) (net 41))
 (segment (start 110.363 86.1295) (end 108.458 88.0345) (width 0.25) (layer F.Cu) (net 41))
 (segment (start 110.363 85.852) (end 110.363 86.1295) (width 0.25) (layer F.Cu) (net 41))
 (segment (start 98.496998 86.995) (end 97.802 86.300002) (width 0.25) (layer F.Cu) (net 41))
 (segment (start 108.1805 88.0345) (end 105.918 90.297) (width 0.25) (layer F.Cu) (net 41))
 (segment (start 105.918 90.297) (end 103.632 90.297) (width 0.25) (layer F.Cu) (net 41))
 (segment (start 97.802 86.300002) (end 97.802 85.815) (width 0.25) (layer F.Cu) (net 41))
 (segment (start 108.458 88.0345) (end 108.1805 88.0345) (width 0.25) (layer F.Cu) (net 41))
 (segment (start 103.632 90.297) (end 103.124 89.789) (width 0.25) (layer F.Cu) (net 41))
 (segment (start 103.124 89.789) (end 103.124 87.63) (width 0.25) (layer F.Cu) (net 41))
 (segment (start 102.489 86.995) (end 98.496998 86.995) (width 0.25) (layer F.Cu) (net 41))
 (segment (start 103.124 87.63) (end 102.489 86.995) (width 0.25) (layer F.Cu) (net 41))
 (segment (start 105.918 71.882) (end 107.315 71.882) (width 0.25) (layer F.Cu) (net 41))
 (segment (start 107.315 71.882) (end 108.077 72.644) (width 0.25) (layer F.Cu) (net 41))
 (segment (start 108.077 72.644) (end 110.236 72.644) (width 0.25) (layer F.Cu) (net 41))
 (segment (start 110.998 71.882) (end 112.638 71.882) (width 0.25) (layer F.Cu) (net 41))
 (segment (start 110.236 72.644) (end 110.998 71.882) (width 0.25) (layer F.Cu) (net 41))
 (segment (start 96.744 69.276) (end 95.062 69.276) (width 0.25) (layer F.Cu) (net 44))
 (segment (start 96.962 69.494) (end 96.744 69.276) (width 0.25) (layer F.Cu) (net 44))
 (segment (start 96.962 70.274) (end 96.962 69.494) (width 0.25) (layer F.Cu) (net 44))
 (segment (start 92.812115 67.281001) (end 93.418116 66.675) (width 0.25) (layer F.Cu) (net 44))
 (segment (start 92.812115 68.929663) (end 92.812115 67.281001) (width 0.25) (layer F.Cu) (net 44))
 (segment (start 93.418116 66.675) (end 94.488 66.675) (width 0.25) (layer F.Cu) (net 44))
 (segment (start 95.062 67.249) (end 95.062 69.53) (width 0.25) (layer F.Cu) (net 44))
 (segment (start 94.488 66.675) (end 95.062 67.249) (width 0.25) (layer F.Cu) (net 44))
 (segment (start 95.062 69.276) (end 95.062 69.53) (width 0.25) (layer F.Cu) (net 44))
 (segment (start 95.062 69.53) (end 95.062 70.274) (width 0.25) (layer F.Cu) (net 44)))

